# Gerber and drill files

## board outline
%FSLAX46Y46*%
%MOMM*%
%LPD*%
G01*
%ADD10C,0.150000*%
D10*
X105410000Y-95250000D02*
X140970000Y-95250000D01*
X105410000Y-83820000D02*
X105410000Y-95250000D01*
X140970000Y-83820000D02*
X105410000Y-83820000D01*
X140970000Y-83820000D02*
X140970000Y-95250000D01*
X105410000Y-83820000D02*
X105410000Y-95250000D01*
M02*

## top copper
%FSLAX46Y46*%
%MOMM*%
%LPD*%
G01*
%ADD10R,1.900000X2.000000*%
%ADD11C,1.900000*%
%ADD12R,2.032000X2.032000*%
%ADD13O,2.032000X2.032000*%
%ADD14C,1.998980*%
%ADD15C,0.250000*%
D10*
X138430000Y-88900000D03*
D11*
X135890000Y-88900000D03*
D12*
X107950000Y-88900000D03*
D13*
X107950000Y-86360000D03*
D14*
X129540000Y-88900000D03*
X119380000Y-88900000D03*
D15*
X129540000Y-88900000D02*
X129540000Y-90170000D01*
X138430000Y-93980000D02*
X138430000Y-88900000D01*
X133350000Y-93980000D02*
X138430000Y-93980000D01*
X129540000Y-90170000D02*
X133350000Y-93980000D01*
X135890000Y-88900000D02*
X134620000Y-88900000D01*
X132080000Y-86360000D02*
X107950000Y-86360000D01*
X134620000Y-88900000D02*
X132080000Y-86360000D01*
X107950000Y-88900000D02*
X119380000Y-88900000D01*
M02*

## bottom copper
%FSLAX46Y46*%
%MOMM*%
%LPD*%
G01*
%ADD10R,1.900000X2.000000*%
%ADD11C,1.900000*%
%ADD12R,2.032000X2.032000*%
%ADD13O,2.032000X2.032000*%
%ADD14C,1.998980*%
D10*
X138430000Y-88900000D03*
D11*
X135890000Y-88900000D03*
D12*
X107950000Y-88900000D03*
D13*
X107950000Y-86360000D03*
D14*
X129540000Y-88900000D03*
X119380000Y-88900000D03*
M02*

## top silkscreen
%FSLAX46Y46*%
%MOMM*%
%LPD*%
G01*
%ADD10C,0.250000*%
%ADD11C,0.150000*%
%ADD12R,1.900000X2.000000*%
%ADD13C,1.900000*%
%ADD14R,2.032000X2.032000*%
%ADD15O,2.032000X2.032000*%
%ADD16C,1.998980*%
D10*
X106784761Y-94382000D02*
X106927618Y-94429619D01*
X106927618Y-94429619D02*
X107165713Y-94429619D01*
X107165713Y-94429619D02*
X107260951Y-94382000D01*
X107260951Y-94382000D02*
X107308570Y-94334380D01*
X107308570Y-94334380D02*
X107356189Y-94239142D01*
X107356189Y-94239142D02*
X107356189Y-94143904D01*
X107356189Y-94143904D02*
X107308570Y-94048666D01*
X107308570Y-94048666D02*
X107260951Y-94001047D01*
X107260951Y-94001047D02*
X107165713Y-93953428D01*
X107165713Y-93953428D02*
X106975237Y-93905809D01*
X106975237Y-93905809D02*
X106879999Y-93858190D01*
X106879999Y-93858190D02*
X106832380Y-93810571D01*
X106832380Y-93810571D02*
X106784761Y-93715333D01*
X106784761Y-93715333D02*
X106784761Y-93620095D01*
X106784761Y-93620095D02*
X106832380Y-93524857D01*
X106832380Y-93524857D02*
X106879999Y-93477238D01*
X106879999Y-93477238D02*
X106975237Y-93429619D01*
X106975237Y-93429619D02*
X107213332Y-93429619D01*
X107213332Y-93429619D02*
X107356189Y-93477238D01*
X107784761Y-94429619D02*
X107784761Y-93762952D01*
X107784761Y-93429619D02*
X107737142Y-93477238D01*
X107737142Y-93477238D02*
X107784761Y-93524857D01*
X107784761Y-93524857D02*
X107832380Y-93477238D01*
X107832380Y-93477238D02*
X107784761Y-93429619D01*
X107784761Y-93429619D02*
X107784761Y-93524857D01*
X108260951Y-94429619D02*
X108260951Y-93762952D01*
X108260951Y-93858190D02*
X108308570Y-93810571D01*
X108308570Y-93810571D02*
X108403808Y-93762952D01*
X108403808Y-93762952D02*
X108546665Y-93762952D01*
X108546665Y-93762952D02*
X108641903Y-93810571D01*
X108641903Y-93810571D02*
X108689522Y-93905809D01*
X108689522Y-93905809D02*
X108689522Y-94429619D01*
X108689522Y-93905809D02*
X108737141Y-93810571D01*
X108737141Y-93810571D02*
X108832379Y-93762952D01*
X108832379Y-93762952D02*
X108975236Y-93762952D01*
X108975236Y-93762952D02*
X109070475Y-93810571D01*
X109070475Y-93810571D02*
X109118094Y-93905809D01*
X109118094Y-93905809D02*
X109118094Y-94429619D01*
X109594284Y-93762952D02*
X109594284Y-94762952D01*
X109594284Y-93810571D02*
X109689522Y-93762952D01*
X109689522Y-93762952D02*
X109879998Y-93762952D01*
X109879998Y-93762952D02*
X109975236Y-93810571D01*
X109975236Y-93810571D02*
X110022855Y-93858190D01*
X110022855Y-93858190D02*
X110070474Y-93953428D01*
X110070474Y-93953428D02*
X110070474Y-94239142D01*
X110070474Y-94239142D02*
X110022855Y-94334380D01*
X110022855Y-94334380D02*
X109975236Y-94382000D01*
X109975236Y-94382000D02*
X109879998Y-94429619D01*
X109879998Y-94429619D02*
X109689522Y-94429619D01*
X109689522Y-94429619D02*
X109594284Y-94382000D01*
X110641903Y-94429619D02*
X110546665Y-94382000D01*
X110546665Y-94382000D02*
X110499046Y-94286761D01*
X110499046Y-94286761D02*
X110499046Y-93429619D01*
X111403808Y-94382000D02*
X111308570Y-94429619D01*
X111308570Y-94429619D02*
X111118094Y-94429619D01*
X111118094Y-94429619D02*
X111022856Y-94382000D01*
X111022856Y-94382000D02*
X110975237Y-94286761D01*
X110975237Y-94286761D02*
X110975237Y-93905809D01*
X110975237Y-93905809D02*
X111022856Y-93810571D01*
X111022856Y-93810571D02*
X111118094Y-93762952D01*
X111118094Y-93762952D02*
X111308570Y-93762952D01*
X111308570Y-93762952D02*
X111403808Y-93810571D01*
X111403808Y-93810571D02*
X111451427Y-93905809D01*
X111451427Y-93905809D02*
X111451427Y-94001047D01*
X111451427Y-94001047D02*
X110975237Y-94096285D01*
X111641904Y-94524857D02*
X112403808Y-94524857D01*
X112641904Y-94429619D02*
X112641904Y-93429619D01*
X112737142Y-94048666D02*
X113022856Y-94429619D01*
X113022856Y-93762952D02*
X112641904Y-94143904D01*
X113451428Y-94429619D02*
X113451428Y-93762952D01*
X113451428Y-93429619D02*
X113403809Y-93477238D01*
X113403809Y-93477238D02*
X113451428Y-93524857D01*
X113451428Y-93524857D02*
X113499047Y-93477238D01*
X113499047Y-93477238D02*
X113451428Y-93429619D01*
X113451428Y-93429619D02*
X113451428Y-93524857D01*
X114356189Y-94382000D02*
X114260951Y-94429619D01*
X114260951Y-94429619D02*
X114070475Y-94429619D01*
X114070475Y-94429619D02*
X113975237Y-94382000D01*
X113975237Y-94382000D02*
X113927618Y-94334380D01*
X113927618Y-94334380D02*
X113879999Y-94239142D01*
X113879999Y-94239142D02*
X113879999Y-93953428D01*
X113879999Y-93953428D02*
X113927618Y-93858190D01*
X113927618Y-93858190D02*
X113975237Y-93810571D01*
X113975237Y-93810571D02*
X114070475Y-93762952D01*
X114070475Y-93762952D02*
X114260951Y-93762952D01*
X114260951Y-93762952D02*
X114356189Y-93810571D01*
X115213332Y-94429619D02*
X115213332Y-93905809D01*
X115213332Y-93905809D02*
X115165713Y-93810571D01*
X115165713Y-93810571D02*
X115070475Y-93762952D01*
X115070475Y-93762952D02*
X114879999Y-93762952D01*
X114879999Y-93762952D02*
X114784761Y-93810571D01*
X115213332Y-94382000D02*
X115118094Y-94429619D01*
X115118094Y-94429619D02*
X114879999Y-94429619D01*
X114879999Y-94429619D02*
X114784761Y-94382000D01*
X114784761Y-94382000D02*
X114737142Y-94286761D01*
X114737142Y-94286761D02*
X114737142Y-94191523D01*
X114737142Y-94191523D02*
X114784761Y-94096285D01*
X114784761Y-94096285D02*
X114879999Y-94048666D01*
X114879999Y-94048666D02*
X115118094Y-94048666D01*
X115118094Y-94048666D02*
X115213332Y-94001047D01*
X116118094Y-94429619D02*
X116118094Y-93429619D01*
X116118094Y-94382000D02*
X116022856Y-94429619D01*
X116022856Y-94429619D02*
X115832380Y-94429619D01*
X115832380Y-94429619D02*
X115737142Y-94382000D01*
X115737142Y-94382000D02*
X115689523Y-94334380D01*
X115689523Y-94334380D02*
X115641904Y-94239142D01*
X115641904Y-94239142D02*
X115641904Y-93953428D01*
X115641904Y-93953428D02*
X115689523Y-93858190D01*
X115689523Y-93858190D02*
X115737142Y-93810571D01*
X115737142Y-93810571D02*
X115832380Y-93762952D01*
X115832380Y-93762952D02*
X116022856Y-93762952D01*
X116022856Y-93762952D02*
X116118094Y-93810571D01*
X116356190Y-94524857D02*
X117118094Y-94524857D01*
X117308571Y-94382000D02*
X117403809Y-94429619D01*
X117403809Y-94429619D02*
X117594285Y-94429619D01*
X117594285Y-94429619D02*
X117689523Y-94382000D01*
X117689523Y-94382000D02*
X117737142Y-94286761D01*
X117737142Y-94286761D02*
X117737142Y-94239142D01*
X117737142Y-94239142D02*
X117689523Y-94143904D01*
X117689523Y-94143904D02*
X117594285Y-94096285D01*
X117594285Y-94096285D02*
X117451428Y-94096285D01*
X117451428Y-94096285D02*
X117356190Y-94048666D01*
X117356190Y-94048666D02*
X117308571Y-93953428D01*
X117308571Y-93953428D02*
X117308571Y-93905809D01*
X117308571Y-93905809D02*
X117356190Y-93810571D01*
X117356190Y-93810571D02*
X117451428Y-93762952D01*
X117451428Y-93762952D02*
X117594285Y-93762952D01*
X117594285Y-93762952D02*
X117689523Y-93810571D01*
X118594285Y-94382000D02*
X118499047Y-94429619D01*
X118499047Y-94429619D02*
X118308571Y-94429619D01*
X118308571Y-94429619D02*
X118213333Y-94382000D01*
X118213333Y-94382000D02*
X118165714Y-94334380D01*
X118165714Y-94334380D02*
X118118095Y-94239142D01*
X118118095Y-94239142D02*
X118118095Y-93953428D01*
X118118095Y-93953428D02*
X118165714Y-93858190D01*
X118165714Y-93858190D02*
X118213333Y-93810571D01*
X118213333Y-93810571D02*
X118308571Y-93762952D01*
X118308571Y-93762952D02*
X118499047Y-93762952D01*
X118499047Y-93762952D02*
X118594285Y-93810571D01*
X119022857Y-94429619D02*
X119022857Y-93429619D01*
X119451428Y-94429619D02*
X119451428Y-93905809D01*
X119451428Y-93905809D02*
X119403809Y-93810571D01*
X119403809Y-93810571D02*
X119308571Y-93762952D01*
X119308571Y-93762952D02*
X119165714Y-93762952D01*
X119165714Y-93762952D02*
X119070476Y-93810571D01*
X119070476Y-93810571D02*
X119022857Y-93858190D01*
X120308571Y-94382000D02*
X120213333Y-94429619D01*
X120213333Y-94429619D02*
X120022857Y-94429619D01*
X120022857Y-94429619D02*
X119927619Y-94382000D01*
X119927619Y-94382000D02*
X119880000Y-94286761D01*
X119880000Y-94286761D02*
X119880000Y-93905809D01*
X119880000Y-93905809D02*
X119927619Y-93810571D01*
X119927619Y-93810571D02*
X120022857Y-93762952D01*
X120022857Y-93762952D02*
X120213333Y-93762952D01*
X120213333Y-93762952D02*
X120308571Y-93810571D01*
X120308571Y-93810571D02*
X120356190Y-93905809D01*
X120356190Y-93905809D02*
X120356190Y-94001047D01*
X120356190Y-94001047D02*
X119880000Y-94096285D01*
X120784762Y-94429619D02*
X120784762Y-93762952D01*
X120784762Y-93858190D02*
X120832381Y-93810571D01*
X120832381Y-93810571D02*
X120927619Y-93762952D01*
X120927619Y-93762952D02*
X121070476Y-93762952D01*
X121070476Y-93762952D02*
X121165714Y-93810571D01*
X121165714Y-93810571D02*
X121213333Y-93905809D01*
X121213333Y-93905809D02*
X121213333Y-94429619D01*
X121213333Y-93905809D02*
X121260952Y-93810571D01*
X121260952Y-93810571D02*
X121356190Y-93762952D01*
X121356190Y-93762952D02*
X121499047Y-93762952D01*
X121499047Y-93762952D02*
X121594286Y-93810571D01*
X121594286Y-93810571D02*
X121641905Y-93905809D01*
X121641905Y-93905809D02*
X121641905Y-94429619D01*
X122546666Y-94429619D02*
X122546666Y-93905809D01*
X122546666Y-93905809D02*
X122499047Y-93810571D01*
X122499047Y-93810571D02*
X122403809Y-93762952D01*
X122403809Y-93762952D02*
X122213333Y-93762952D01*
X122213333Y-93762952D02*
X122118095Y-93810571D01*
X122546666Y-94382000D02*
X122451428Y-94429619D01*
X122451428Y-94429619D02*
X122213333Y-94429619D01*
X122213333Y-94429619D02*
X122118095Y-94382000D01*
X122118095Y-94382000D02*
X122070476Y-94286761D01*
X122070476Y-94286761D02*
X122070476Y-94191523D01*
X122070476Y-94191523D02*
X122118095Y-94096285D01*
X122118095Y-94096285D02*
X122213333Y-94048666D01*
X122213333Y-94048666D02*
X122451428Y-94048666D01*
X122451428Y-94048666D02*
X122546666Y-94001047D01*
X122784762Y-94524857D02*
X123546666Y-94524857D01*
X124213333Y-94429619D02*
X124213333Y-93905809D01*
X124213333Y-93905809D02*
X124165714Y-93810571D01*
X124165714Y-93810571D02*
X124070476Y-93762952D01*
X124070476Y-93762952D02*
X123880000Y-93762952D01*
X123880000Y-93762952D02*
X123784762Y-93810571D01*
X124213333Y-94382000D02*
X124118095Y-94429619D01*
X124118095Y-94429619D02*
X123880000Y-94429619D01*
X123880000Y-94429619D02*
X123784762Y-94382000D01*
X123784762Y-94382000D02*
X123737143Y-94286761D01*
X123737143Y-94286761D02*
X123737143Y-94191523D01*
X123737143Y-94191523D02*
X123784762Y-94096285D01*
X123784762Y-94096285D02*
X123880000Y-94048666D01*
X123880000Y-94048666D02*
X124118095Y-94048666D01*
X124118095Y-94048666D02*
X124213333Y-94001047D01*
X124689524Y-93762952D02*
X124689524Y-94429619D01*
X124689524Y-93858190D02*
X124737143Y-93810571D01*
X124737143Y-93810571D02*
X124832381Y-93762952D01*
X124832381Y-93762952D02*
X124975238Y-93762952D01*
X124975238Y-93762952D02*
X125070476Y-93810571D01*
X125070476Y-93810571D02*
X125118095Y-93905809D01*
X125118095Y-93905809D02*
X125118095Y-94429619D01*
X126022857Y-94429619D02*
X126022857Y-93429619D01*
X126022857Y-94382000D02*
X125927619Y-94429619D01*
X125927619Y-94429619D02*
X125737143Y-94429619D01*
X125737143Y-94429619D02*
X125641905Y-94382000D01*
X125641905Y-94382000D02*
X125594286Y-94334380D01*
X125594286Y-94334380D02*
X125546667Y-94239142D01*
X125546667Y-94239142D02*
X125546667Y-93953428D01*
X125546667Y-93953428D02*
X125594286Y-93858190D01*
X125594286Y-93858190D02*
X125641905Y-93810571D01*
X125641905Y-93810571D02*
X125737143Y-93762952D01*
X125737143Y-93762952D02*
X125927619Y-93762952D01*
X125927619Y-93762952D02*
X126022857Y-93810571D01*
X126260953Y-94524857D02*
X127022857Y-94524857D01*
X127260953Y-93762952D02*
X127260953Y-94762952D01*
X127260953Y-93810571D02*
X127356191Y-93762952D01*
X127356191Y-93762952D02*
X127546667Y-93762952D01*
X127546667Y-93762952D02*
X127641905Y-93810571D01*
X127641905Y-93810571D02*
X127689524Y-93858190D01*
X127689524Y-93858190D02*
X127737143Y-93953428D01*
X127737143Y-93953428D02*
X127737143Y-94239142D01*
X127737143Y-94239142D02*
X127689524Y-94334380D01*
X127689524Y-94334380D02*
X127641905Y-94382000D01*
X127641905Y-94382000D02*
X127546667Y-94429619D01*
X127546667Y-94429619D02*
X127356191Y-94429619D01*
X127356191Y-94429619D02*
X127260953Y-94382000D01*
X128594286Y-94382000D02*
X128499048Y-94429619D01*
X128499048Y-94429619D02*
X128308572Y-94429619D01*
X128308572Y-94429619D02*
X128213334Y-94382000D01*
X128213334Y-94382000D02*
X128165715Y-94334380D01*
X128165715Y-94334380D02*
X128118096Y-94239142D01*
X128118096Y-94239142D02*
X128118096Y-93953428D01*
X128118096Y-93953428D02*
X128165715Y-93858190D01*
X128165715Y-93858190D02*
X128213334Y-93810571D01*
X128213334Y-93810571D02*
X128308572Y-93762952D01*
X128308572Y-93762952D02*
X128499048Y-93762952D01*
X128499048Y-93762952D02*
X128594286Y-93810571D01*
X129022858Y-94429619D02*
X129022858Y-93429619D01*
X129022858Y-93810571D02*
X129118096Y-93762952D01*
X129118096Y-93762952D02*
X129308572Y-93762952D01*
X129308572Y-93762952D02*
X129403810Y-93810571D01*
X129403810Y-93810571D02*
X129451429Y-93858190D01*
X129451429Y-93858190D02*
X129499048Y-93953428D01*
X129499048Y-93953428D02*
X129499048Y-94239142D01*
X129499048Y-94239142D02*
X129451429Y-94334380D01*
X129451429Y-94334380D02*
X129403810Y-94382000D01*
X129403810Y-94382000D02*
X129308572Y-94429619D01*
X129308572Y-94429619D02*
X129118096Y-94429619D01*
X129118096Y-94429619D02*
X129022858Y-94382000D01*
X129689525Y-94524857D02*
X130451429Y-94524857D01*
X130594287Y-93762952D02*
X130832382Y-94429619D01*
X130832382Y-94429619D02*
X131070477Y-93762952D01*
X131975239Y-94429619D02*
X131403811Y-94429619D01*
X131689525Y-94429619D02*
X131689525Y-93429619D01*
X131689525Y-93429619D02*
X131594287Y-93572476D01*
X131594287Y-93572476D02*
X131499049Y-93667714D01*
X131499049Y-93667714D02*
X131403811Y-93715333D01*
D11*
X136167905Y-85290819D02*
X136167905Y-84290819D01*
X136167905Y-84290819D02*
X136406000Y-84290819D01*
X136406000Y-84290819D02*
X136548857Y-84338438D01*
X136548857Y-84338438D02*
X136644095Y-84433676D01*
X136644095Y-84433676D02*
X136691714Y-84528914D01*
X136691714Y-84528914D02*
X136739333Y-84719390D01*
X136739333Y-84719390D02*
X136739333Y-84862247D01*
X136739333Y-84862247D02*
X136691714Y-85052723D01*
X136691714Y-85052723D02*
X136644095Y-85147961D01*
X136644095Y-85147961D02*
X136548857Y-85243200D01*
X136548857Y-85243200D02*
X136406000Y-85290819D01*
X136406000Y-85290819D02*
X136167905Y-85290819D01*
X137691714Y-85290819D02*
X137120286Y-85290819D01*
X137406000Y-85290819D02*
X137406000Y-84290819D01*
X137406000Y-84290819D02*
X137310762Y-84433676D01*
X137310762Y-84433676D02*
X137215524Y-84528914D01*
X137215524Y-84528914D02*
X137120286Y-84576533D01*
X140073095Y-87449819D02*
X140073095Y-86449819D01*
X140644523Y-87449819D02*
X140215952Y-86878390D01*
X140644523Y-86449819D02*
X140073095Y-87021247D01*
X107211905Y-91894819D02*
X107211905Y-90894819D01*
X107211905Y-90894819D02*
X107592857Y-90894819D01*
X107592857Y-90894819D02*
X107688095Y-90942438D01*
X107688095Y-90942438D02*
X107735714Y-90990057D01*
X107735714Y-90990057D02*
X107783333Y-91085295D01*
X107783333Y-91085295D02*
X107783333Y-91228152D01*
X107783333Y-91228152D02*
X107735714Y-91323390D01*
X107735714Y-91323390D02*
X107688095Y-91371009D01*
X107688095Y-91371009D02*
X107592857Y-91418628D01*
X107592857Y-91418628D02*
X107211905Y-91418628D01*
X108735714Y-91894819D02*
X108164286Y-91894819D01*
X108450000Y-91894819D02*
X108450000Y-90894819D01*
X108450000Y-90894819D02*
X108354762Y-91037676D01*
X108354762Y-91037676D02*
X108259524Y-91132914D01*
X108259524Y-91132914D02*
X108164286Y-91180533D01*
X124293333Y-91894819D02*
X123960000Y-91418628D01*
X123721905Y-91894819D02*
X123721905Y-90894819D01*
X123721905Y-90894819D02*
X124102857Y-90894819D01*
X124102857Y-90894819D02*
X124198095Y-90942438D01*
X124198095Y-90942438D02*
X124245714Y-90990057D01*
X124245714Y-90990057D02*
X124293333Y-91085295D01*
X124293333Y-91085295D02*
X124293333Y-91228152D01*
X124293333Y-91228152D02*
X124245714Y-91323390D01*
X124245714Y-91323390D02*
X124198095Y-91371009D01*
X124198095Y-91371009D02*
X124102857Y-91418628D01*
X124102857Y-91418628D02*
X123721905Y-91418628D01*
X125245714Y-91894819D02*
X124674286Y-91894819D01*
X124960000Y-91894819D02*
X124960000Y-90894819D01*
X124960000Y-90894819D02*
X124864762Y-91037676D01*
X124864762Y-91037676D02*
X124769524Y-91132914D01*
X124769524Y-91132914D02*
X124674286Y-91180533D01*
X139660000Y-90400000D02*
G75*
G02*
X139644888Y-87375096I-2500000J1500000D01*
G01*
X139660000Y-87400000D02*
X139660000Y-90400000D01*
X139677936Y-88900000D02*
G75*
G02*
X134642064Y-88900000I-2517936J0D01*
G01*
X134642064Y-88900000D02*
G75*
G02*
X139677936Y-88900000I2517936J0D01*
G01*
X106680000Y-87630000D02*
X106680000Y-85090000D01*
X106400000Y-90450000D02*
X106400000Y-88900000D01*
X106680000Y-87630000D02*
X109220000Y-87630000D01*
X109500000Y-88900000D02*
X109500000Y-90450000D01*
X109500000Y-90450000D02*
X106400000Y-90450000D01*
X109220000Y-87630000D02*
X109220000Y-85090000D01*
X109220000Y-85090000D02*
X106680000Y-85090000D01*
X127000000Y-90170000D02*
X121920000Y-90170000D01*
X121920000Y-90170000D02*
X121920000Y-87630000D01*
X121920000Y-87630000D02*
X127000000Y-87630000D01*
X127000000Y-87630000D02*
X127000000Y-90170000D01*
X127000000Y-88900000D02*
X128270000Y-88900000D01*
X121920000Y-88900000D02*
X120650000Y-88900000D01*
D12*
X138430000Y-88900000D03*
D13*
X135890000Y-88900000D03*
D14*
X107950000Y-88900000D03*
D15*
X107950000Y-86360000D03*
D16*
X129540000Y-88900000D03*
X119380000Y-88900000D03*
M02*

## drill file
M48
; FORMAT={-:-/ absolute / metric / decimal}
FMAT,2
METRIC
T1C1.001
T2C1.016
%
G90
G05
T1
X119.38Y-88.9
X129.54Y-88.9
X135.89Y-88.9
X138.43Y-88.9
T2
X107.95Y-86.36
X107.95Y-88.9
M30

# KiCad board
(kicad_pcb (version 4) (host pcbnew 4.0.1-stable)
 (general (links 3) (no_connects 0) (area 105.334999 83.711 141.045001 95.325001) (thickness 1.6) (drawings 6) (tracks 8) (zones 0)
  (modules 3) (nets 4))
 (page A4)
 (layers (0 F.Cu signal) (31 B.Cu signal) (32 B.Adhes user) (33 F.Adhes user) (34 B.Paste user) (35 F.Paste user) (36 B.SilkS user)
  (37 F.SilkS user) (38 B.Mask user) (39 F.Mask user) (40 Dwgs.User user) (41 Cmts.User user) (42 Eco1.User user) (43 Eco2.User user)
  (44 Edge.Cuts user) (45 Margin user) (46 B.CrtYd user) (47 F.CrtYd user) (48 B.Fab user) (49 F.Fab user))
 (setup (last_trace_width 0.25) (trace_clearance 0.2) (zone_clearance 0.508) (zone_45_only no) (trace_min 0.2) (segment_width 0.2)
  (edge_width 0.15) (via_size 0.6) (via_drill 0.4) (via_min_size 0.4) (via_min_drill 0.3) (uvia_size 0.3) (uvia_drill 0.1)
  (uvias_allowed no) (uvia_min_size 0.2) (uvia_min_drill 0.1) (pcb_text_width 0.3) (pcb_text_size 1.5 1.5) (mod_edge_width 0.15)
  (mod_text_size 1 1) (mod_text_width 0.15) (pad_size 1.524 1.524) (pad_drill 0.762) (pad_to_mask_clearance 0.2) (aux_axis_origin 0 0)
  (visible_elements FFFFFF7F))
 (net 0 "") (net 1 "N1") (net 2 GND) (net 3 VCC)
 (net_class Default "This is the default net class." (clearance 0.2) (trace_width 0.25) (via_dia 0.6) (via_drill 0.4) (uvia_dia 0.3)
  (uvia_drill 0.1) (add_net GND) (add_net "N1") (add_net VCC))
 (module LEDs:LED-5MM (layer F.Cu) (at 138.43 88.9 180)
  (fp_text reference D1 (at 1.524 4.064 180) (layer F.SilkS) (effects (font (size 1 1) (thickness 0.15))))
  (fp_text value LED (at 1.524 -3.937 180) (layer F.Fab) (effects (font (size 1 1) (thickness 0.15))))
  (fp_arc (start 1.27 0) (end -1.23 -1.5) (angle 297.5) (layer F.SilkS) (width 0.15))
  (fp_line (start -1.23 1.5) (end -1.23 -1.5) (layer F.SilkS) (width 0.15))
  (fp_circle (center 1.27 0) (end 0.97 -2.5) (layer F.SilkS) (width 0.15))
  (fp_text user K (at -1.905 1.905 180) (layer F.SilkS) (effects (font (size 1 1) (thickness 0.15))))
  (pad 1 thru_hole rect (at 0 0 270) (size 2 1.9) (drill 1.00076) (layers *.Cu *.Mask F.SilkS) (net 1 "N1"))
  (pad 2 thru_hole circle (at 2.54 0 180) (size 1.9 1.9) (drill 1.00076) (layers *.Cu *.Mask F.SilkS) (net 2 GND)))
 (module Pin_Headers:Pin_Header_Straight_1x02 (layer F.Cu) (at 107.95 88.9 180)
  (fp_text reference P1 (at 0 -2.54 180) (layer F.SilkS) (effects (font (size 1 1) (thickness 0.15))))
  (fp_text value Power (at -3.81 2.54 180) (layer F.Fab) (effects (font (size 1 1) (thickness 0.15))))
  (fp_line (start 1.27 1.27) (end 1.27 3.81) (layer F.SilkS) (width 0.15))
  (fp_line (start 1.55 -1.55) (end 1.55 0) (layer F.SilkS) (width 0.15))
  (fp_line (start 1.27 1.27) (end -1.27 1.27) (layer F.SilkS) (width 0.15))
  (fp_line (start -1.55 0) (end -1.55 -1.55) (layer F.SilkS) (width 0.15))
  (fp_line (start -1.55 -1.55) (end 1.55 -1.55) (layer F.SilkS) (width 0.15))
  (fp_line (start -1.27 1.27) (end -1.27 3.81) (layer F.SilkS) (width 0.15))
  (fp_line (start -1.27 3.81) (end 1.27 3.81) (layer F.SilkS) (width 0.15))
  (pad 1 thru_hole rect (at 0 0 180) (size 2.032 2.032) (drill 1.016) (layers *.Cu *.Mask F.SilkS) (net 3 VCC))
  (pad 2 thru_hole oval (at 0 2.54 180) (size 2.032 2.032) (drill 1.016) (layers *.Cu *.Mask F.SilkS) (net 2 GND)))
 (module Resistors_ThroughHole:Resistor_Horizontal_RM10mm (layer F.Cu) (at 124.46 88.9 180)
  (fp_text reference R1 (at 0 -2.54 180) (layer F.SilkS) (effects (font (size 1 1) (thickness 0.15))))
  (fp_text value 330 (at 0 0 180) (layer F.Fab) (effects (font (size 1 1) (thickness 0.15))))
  (fp_line (start -2.54 -1.27) (end 2.54 -1.27) (layer F.SilkS) (width 0.15))
  (fp_line (start 2.54 -1.27) (end 2.54 1.27) (layer F.SilkS) (width 0.15))
  (fp_line (start 2.54 1.27) (end -2.54 1.27) (layer F.SilkS) (width 0.15))
  (fp_line (start -2.54 1.27) (end -2.54 -1.27) (layer F.SilkS) (width 0.15))
  (fp_line (start -2.54 0) (end -3.81 0) (layer F.SilkS) (width 0.15))
  (fp_line (start 2.54 0) (end 3.81 0) (layer F.SilkS) (width 0.15))
  (pad 1 thru_hole circle (at -5.08 0 180) (size 1.99898 1.99898) (drill 1.00076) (layers *.Cu *.SilkS *.Mask) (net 1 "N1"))
  (pad 2 thru_hole circle (at 5.08 0 180) (size 1.99898 1.99898) (drill 1.00076) (layers *.Cu *.SilkS *.Mask) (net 3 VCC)))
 (gr_line (start 105.41 95.25) (end 140.97 95.25) (angle 90) (layer Edge.Cuts) (width 0.15))
 (gr_line (start 105.41 83.82) (end 105.41 95.25) (angle 90) (layer Edge.Cuts) (width 0.15))
 (gr_line (start 140.97 83.82) (end 105.41 83.82) (angle 90) (layer Edge.Cuts) (width 0.15))
 (gr_line (start 140.97 83.82) (end 140.97 95.25) (angle 90) (layer Edge.Cuts) (width 0.15))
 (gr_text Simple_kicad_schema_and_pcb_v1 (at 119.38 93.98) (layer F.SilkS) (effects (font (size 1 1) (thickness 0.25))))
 (gr_line (start 105.41 83.82) (end 105.41 95.25) (angle 90) (layer Edge.Cuts) (width 0.15))
 (segment (start 129.54 88.9) (end 129.54 90.17) (width 0.25) (layer F.Cu) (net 1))
 (segment (start 138.43 93.98) (end 138.43 88.9) (width 0.25) (layer F.Cu) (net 1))
 (segment (start 133.35 93.98) (end 138.43 93.98) (width 0.25) (layer F.Cu) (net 1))
 (segment (start 129.54 90.17) (end 133.35 93.98) (width 0.25) (layer F.Cu) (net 1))
 (segment (start 135.89 88.9) (end 134.62 88.9) (width 0.25) (layer F.Cu) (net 2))
 (segment (start 132.08 86.36) (end 107.95 86.36) (width 0.25) (layer F.Cu) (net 2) (status 20))
 (segment (start 134.62 88.9) (end 132.08 86.36) (width 0.25) (layer F.Cu) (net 2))
 (segment (start 107.95 88.9) (end 119.38 88.9) (width 0.25) (layer F.Cu) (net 3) (status 10)))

